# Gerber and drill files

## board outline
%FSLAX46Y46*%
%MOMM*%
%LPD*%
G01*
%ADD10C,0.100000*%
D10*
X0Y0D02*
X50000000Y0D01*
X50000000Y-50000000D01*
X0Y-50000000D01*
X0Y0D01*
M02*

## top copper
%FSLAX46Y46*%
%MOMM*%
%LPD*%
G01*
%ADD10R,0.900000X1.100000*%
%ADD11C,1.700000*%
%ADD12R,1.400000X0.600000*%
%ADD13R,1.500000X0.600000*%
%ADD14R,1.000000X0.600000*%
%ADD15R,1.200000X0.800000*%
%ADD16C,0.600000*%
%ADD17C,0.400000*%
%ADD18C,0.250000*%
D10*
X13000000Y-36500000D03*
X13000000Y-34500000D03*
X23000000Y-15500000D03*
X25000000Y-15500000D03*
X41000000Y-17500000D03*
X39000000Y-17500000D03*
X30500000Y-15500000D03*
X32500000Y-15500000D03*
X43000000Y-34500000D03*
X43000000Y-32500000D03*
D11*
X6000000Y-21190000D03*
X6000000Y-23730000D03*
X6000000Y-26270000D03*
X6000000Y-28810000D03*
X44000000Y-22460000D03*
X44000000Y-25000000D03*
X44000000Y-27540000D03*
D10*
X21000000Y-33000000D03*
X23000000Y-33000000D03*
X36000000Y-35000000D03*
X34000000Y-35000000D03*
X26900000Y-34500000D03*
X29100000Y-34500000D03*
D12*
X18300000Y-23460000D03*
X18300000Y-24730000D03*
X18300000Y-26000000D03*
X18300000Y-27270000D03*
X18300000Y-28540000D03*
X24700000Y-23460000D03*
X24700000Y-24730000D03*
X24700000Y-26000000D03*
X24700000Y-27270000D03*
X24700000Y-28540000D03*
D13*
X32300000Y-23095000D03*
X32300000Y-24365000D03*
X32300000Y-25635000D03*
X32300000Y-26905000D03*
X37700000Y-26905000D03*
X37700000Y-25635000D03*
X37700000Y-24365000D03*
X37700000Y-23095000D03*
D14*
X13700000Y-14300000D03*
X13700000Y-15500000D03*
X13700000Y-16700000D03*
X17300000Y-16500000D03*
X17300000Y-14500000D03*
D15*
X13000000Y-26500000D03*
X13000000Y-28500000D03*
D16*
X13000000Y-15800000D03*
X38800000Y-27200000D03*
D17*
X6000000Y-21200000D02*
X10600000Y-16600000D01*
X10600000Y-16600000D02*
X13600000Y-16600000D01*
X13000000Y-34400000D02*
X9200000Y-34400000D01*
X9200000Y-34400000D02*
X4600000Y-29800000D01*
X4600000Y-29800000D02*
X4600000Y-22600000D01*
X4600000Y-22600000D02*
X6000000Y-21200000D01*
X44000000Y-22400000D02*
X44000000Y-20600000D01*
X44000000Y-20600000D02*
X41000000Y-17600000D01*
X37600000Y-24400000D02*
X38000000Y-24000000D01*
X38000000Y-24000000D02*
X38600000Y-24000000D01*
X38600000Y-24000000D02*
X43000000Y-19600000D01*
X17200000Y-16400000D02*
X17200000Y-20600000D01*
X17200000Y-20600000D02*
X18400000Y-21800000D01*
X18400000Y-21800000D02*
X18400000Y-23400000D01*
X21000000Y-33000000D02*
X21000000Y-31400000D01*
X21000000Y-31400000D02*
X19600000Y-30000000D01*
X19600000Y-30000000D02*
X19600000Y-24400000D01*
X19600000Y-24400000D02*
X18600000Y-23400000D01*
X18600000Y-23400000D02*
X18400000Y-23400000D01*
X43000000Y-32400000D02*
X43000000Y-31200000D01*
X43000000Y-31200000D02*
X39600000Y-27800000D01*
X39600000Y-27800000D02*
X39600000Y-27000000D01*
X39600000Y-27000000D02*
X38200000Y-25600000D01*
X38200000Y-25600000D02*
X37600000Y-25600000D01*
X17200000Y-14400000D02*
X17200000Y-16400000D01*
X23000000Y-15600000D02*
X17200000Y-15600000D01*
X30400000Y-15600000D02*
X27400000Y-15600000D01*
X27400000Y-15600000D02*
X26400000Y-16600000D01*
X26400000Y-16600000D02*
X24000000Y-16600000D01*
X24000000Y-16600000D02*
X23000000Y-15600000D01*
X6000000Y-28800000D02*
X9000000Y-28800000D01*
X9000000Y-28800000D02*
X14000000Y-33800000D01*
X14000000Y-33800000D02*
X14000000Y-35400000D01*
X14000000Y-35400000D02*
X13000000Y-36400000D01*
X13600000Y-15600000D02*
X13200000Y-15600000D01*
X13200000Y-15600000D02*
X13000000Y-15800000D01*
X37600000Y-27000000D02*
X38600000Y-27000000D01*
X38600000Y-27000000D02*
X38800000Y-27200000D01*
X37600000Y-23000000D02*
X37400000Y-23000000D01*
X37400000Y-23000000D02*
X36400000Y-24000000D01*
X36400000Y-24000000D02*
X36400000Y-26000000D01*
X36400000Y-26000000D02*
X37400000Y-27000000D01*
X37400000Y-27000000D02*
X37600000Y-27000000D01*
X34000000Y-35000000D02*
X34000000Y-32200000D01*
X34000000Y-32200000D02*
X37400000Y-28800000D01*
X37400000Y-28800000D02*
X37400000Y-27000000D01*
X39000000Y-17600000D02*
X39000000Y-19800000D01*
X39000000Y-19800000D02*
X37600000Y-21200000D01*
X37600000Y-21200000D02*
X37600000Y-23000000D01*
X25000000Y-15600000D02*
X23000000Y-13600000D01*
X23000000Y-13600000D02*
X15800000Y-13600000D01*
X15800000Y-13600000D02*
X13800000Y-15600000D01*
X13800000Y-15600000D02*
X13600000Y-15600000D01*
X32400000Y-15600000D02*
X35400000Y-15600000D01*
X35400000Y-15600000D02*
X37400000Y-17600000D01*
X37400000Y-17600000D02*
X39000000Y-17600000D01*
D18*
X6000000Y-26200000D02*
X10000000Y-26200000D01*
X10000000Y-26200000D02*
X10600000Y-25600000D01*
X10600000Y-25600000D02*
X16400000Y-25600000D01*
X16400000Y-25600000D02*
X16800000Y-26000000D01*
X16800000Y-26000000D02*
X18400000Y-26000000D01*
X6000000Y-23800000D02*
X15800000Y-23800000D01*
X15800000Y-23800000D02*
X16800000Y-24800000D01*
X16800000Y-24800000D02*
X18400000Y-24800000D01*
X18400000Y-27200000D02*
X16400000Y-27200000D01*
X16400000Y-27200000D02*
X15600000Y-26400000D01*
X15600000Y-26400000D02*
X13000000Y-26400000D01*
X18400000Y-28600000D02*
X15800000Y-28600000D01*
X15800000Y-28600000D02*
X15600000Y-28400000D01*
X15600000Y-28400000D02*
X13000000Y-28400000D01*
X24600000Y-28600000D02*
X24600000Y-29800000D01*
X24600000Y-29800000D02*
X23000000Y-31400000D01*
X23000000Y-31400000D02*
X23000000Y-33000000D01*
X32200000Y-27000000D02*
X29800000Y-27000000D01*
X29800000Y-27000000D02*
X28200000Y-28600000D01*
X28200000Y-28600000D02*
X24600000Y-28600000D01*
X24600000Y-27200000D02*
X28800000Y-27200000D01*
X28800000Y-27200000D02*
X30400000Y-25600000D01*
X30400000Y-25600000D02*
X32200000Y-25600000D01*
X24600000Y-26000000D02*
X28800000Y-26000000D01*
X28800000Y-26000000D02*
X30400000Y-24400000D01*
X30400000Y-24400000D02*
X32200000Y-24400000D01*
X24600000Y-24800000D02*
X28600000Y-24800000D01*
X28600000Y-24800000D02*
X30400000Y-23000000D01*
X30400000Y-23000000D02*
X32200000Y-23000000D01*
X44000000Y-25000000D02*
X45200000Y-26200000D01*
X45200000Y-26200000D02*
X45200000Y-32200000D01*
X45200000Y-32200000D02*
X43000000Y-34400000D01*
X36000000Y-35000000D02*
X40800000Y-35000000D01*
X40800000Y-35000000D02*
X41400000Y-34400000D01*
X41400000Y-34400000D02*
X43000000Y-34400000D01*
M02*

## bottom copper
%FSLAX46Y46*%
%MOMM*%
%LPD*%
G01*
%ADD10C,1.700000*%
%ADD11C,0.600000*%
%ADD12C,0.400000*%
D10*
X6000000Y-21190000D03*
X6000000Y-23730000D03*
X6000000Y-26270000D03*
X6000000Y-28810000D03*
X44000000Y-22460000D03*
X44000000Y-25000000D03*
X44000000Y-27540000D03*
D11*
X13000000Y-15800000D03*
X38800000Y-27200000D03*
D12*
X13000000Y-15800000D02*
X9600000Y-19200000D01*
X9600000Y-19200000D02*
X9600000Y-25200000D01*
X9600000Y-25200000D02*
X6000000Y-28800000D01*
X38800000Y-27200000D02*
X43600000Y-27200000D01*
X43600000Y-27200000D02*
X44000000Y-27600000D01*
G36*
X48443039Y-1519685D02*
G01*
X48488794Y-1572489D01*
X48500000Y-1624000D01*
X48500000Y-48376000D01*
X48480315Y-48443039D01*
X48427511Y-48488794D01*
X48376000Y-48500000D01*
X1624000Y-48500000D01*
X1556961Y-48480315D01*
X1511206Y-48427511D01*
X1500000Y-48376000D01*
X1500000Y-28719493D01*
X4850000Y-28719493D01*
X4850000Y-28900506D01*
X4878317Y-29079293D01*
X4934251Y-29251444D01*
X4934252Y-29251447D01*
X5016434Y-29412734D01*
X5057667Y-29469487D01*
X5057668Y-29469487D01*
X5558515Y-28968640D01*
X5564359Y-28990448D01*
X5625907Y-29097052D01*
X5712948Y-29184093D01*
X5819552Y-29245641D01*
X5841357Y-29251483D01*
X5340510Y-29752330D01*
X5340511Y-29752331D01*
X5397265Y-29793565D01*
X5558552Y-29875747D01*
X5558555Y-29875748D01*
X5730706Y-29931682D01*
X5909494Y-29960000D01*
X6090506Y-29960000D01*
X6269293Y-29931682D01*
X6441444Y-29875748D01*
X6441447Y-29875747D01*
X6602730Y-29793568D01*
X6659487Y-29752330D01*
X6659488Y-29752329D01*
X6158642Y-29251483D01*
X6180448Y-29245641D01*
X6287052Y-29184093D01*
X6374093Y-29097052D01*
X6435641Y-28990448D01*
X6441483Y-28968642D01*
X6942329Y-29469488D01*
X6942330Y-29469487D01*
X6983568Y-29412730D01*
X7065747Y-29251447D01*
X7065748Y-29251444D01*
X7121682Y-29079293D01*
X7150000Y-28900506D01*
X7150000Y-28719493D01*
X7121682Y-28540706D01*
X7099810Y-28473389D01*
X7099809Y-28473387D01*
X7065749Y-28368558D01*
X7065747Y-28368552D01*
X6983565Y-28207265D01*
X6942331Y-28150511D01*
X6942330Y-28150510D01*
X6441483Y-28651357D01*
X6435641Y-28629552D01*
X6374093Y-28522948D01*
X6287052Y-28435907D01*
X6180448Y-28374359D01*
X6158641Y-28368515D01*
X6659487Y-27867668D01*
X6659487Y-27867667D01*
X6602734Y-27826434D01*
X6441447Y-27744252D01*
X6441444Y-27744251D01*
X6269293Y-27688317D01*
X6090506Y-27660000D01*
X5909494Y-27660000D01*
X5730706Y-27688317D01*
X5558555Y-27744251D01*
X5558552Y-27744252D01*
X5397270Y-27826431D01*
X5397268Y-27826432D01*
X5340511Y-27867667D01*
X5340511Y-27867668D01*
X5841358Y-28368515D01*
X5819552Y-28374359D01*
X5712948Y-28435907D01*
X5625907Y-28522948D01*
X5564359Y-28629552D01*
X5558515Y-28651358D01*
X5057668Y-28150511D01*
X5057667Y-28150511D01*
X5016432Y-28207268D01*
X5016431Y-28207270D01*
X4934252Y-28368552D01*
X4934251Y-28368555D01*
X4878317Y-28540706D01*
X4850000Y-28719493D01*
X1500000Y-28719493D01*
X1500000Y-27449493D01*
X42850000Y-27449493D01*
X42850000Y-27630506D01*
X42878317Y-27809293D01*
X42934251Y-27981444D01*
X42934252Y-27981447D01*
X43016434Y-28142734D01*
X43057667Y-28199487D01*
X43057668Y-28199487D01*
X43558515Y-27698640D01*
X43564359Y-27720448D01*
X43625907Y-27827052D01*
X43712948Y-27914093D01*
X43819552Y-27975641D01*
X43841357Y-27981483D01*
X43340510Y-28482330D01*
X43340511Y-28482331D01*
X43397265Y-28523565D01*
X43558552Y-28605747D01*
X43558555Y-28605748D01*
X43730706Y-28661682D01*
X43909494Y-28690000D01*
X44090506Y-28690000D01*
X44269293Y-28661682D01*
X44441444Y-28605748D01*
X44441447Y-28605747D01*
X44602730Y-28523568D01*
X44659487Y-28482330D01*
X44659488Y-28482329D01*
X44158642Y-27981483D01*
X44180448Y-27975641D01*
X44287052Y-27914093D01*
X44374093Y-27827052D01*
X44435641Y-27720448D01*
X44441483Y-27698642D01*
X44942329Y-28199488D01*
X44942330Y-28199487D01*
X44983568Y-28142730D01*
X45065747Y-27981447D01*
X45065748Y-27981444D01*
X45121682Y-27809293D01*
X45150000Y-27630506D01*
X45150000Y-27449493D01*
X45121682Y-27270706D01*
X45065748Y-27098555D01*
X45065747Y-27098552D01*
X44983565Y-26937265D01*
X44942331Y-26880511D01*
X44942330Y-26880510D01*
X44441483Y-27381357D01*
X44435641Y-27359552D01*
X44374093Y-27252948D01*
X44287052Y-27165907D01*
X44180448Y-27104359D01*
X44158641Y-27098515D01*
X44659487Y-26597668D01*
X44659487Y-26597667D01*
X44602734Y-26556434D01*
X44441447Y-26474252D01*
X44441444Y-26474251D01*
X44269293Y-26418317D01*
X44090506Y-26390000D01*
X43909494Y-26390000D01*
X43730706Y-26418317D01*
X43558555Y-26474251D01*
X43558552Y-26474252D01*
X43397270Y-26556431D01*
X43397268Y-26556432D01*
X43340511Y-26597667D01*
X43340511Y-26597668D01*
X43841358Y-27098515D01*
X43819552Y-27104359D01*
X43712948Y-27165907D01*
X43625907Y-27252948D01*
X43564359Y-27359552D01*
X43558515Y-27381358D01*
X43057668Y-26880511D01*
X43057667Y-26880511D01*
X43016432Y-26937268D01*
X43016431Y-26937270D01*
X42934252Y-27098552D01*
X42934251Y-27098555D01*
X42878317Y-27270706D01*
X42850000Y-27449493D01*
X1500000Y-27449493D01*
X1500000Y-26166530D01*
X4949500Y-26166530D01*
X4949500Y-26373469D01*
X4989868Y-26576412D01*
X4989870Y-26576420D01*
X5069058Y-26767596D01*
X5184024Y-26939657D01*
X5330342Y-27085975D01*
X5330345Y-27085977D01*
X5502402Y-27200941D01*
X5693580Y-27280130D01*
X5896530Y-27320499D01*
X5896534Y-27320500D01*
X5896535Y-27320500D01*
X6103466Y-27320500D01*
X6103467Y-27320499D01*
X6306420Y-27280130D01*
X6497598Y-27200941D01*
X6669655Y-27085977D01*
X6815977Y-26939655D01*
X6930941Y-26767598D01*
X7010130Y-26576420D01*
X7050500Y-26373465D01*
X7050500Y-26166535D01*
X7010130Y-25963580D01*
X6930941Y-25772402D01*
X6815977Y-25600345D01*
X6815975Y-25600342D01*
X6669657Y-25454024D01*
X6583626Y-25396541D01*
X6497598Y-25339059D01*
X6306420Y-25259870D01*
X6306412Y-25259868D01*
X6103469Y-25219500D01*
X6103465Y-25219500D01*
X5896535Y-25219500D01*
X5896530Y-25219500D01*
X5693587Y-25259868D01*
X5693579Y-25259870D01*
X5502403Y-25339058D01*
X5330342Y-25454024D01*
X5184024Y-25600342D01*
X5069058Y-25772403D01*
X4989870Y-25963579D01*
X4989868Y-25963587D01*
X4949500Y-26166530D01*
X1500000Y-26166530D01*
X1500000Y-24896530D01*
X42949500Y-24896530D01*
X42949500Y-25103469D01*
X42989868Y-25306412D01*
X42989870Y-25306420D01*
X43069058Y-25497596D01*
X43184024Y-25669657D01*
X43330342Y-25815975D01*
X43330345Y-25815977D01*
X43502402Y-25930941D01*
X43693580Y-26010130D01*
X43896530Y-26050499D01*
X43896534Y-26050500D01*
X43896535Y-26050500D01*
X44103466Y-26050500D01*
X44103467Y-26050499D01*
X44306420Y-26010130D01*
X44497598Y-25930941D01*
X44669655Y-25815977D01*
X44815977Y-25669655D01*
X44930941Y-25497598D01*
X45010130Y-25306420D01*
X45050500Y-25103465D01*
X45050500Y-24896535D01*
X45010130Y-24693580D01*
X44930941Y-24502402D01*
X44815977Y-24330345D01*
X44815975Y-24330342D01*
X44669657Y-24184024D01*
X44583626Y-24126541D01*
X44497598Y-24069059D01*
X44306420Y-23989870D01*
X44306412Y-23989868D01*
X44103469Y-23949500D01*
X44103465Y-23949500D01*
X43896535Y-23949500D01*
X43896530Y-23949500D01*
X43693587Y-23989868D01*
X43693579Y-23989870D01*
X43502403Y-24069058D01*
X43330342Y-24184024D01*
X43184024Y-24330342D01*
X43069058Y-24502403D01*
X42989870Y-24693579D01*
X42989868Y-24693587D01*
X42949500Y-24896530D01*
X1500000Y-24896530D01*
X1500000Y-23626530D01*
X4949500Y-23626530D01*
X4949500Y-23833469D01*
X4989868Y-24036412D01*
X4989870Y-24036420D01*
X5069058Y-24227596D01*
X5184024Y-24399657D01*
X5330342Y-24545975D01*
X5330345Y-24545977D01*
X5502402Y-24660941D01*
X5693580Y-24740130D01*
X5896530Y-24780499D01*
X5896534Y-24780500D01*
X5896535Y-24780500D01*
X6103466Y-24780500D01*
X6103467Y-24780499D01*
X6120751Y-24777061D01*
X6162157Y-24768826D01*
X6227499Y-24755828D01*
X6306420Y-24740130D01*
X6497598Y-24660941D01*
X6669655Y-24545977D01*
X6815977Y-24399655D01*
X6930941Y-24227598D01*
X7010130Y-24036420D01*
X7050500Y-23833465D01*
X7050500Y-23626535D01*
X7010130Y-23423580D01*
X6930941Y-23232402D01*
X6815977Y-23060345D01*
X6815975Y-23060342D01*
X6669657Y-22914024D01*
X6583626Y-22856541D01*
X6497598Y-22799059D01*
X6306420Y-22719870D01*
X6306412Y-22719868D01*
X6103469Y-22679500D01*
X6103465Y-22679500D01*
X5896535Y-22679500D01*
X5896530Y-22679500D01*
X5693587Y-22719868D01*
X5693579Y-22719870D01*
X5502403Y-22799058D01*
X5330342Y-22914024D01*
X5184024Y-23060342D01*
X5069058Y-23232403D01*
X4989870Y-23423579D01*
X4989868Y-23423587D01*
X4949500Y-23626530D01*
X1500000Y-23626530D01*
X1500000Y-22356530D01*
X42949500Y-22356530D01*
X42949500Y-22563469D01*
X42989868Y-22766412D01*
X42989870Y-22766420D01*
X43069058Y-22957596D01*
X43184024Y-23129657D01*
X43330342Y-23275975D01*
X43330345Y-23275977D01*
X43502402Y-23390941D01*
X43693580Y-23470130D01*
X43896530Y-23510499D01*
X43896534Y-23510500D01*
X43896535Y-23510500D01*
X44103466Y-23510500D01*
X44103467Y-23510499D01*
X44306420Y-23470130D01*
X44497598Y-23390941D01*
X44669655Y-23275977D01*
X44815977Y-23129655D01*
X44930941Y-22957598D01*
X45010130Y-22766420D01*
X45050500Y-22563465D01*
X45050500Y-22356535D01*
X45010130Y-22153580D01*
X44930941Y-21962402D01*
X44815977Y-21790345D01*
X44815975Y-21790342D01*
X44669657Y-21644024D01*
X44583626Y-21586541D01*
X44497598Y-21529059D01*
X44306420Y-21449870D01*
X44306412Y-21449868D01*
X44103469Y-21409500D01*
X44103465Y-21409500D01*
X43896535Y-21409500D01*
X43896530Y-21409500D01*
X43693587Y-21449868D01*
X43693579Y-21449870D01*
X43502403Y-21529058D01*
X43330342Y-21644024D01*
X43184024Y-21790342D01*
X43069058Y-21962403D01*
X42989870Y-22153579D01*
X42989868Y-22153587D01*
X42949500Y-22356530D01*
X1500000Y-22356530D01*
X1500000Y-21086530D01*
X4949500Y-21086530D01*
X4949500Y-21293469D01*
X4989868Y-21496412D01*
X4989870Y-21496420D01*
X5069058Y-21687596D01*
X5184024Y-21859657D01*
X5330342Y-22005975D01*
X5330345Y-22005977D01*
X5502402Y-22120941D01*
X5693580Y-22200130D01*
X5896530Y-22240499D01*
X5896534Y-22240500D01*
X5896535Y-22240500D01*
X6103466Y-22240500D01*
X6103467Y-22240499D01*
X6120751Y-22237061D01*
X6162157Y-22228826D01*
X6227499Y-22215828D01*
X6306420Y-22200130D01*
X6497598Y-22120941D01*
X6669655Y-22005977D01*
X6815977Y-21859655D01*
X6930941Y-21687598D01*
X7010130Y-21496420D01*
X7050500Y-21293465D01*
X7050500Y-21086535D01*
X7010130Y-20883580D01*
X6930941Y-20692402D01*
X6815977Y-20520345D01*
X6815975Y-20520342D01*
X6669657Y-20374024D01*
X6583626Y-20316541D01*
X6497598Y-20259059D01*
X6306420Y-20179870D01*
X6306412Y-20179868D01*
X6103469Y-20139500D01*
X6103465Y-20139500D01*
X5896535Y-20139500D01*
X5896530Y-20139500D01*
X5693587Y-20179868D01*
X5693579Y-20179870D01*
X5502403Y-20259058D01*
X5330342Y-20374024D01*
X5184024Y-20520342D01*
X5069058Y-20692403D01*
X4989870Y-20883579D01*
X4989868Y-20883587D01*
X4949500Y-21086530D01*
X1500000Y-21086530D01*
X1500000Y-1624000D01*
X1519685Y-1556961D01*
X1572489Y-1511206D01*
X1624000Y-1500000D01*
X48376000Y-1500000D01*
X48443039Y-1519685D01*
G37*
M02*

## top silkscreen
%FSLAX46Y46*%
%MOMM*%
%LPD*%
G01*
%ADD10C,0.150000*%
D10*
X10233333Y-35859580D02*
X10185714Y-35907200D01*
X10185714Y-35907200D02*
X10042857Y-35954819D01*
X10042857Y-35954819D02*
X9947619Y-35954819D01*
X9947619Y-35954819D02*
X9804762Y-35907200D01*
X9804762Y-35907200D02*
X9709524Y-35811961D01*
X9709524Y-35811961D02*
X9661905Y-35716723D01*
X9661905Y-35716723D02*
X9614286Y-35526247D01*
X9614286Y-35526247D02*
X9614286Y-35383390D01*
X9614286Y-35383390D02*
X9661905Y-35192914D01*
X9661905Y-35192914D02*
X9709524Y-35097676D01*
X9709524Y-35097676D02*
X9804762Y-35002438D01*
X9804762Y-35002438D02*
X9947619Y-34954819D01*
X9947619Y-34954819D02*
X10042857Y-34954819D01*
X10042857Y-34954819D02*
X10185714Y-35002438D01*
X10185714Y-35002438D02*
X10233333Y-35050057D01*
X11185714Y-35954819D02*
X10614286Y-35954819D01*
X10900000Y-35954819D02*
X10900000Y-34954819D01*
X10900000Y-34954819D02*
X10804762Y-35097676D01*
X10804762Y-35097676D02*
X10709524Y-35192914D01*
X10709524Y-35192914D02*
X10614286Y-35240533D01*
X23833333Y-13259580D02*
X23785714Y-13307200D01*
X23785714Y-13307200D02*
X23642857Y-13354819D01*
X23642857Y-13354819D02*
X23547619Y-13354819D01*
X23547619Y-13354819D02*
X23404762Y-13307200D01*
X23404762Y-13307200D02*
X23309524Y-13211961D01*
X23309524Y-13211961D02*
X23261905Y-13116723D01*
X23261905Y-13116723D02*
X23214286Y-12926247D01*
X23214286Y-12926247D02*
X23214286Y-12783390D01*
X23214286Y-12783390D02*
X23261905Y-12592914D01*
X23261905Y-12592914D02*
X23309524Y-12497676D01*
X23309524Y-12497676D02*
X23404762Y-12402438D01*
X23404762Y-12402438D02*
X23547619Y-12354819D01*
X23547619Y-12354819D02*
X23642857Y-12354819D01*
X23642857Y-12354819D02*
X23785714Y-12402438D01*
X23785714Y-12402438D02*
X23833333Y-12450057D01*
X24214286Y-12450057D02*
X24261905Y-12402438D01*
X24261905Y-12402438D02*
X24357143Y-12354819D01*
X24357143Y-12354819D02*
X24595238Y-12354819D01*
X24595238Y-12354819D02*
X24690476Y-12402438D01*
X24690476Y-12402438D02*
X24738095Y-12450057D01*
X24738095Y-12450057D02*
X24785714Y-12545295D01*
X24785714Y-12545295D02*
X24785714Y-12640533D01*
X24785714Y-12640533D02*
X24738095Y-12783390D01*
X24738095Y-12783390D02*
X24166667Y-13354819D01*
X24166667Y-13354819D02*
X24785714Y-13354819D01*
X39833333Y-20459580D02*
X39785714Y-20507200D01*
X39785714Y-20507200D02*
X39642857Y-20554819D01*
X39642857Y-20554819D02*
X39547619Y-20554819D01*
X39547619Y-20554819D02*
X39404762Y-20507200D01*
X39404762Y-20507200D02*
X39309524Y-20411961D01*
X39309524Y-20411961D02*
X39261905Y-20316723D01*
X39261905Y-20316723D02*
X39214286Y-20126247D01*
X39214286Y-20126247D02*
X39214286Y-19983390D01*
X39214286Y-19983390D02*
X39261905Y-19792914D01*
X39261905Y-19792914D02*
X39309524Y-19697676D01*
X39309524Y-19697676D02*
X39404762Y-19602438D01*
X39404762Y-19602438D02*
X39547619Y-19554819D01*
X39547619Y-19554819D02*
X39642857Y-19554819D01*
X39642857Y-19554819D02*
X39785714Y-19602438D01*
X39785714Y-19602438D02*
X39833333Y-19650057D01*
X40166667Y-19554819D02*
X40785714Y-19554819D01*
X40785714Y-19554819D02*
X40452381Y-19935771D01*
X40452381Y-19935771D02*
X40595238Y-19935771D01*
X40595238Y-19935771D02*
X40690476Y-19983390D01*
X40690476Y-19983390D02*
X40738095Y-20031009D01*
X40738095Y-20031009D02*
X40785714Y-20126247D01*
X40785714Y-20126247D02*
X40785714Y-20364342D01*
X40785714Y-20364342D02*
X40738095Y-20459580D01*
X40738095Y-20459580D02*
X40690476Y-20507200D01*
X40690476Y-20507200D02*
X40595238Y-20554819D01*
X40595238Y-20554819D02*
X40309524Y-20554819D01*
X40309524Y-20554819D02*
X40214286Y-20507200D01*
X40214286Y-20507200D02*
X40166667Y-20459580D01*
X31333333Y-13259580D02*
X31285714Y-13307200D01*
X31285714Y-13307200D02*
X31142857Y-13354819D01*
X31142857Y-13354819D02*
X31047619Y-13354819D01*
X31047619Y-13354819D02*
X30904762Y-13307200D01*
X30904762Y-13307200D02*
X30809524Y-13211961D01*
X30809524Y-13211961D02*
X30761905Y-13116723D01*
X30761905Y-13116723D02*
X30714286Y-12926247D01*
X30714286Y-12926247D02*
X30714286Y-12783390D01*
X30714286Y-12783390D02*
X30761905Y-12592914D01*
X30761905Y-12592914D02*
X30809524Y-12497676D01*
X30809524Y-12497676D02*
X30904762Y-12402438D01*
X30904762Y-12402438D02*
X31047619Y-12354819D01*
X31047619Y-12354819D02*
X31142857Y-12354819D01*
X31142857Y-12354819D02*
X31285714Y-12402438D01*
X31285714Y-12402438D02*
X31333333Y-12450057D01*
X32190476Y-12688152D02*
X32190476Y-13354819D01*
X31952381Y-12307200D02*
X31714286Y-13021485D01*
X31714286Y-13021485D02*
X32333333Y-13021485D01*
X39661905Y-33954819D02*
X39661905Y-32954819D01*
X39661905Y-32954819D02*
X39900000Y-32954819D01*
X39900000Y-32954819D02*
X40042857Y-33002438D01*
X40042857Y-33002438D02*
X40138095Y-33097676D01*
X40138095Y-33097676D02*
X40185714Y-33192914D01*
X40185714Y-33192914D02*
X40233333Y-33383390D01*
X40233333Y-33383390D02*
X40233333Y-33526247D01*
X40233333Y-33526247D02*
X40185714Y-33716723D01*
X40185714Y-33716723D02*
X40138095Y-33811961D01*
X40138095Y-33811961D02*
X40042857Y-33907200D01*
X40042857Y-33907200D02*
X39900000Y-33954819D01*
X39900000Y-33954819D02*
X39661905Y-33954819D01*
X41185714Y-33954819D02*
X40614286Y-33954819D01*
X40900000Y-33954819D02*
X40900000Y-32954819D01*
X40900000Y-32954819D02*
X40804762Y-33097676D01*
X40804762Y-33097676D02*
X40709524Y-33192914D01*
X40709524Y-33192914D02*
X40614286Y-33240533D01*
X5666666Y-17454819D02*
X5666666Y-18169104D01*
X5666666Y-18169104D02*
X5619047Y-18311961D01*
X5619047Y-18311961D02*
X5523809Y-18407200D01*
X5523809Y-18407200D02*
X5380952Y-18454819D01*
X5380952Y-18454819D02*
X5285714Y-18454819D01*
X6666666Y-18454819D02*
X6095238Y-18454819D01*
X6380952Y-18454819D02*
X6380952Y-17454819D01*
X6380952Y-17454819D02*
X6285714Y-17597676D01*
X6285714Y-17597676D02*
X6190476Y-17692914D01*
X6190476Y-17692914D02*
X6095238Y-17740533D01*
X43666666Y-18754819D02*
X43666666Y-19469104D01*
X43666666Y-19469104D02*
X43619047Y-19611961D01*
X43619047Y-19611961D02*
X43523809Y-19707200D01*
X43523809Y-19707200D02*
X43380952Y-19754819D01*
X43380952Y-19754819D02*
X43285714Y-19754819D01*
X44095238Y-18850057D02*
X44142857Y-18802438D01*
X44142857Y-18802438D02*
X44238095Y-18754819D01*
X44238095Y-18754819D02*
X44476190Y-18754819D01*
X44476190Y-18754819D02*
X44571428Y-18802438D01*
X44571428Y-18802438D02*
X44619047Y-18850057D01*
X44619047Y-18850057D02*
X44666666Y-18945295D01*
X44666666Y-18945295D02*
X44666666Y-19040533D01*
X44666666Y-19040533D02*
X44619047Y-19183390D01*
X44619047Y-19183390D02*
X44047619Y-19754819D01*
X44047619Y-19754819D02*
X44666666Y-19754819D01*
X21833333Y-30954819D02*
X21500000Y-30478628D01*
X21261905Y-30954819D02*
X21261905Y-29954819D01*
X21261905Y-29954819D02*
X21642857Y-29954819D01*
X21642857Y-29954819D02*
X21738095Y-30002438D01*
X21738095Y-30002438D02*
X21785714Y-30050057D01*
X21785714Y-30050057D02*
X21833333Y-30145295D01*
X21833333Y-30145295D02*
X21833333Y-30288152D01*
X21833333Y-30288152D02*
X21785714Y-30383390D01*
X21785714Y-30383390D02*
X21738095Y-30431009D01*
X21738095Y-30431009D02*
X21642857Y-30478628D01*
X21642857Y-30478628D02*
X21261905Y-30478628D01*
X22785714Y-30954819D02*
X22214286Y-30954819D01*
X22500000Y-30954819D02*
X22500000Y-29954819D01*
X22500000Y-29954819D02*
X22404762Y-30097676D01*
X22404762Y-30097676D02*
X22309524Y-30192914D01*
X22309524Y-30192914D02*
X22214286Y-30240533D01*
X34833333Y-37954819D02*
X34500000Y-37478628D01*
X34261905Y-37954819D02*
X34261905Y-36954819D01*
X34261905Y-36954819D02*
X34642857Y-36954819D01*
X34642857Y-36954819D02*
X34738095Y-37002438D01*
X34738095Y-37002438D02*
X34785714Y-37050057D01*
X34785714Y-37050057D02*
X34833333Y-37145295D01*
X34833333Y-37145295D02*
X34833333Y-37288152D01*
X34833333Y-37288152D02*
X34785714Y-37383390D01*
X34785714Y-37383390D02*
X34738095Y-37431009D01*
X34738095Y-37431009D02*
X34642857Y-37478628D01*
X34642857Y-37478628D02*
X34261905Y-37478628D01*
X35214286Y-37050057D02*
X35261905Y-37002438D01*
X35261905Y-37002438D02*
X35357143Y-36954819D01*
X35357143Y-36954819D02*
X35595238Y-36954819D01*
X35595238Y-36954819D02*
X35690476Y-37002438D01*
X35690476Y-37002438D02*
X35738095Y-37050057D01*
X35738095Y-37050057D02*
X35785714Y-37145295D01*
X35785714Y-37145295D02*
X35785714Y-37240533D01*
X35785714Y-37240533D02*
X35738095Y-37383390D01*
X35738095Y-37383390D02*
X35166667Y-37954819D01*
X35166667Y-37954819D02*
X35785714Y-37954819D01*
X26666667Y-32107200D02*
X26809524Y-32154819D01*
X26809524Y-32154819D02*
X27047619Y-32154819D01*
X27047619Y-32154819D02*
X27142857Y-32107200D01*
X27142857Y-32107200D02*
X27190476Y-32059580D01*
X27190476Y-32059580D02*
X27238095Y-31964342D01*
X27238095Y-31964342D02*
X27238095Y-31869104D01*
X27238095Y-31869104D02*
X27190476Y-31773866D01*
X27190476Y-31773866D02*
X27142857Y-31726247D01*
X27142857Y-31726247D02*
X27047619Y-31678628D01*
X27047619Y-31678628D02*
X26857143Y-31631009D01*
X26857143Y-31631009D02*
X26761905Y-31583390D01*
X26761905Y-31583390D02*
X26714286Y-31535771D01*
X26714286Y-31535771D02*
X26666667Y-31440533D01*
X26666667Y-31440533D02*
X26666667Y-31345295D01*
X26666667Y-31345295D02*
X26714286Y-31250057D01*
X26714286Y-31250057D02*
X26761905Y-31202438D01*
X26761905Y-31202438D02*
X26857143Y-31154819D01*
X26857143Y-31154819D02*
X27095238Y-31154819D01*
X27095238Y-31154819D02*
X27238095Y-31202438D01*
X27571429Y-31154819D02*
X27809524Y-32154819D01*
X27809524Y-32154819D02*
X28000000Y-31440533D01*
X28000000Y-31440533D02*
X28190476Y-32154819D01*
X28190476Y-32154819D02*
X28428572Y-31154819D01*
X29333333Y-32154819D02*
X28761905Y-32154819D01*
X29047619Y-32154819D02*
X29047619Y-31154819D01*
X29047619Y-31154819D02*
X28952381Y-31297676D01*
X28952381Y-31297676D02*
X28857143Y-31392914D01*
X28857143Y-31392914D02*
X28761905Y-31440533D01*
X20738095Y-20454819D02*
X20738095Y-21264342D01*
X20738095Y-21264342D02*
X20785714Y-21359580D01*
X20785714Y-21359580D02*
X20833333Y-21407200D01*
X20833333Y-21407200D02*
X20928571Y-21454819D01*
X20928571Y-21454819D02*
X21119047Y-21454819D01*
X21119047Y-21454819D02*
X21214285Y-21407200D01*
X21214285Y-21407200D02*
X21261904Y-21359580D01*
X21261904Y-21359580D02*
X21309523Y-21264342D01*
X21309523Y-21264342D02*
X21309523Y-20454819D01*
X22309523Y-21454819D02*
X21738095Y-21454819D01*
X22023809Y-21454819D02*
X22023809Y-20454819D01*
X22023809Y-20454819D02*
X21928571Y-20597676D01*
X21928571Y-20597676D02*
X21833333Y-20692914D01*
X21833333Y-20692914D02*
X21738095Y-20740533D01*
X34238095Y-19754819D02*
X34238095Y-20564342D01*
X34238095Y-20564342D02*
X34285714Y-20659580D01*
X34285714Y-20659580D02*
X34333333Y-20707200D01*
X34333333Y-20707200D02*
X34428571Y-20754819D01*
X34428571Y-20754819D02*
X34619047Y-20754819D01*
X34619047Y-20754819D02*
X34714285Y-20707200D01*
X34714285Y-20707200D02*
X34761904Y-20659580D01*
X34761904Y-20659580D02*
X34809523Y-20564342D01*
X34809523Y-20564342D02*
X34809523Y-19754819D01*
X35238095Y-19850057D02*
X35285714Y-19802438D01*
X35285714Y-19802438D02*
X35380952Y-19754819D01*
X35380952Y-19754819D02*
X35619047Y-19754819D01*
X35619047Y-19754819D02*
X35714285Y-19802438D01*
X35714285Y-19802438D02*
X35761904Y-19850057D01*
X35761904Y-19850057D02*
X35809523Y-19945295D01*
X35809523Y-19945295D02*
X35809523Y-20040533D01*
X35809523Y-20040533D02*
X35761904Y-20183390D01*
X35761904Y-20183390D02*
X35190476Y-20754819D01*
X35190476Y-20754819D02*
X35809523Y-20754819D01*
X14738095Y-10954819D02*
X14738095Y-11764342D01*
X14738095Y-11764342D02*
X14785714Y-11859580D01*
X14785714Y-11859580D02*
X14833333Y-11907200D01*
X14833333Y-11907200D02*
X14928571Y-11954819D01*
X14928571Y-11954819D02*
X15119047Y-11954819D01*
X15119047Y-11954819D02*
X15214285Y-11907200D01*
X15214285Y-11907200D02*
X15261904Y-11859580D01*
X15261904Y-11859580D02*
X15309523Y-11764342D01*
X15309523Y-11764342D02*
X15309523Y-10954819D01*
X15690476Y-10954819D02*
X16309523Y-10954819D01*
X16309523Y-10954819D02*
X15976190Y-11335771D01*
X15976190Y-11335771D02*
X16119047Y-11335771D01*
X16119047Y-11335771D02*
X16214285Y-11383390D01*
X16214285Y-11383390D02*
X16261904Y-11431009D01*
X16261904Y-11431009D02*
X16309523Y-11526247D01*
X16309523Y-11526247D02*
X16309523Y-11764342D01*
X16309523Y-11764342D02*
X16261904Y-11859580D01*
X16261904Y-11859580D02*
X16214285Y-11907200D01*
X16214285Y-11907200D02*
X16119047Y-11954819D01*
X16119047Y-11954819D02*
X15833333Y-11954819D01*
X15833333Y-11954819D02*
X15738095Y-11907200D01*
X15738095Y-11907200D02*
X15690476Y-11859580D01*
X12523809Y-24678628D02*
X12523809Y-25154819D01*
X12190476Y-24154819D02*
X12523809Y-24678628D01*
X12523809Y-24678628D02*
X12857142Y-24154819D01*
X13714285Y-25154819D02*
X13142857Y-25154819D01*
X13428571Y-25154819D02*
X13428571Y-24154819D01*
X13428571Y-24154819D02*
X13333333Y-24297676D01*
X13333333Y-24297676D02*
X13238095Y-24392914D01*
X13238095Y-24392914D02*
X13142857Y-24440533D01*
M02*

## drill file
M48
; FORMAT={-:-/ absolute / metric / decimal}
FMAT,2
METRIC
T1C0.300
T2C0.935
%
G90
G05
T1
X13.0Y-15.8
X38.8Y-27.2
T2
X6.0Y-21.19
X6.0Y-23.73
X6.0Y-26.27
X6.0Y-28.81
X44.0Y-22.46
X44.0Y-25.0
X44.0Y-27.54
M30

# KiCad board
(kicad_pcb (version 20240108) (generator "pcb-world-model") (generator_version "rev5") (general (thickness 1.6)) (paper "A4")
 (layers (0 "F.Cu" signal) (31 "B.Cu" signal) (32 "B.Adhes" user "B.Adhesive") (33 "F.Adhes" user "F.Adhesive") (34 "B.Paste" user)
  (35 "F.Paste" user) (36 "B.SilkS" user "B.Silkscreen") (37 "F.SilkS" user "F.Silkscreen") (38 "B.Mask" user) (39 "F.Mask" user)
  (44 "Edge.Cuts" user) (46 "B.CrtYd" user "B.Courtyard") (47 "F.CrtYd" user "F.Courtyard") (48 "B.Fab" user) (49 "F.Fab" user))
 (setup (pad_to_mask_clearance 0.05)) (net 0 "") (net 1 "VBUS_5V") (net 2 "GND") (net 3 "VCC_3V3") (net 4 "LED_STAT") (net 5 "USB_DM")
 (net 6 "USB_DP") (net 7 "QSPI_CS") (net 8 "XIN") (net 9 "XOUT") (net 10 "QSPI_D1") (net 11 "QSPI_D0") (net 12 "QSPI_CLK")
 (gr_rect (start 0.0 0.0) (end 50.0000 50.0000) (stroke (width 0.1) (type default)) (fill none) (layer "Edge.Cuts"))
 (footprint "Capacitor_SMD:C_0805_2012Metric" (layer "F.Cu") (at 13.0000 35.5000 90)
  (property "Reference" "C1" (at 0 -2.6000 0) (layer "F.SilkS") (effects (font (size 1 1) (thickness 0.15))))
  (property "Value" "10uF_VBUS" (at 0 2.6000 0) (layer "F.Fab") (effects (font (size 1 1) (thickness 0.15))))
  (pad "1" smd rect (at -1.0000 0.0000) (size 0.9000 1.1000) (layers "F.Cu" "F.Paste" "F.Mask") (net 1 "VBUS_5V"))
  (pad "2" smd rect (at 1.0000 0.0000) (size 0.9000 1.1000) (layers "F.Cu" "F.Paste" "F.Mask") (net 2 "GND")))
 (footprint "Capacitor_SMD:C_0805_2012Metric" (layer "F.Cu") (at 24.0000 15.5000 0)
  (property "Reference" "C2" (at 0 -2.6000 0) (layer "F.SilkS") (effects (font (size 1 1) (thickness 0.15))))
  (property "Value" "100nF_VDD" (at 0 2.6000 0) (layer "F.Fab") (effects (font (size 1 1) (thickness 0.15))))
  (pad "1" smd rect (at -1.0000 0.0000) (size 0.9000 1.1000) (layers "F.Cu" "F.Paste" "F.Mask") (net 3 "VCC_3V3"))
  (pad "2" smd rect (at 1.0000 0.0000) (size 0.9000 1.1000) (layers "F.Cu" "F.Paste" "F.Mask") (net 2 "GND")))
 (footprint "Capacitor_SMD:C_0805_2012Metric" (layer "F.Cu") (at 40.0000 17.5000 180)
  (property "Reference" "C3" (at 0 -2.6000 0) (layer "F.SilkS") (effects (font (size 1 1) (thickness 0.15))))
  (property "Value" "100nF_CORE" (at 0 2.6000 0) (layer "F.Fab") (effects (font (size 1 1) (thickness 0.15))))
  (pad "1" smd rect (at -1.0000 0.0000) (size 0.9000 1.1000) (layers "F.Cu" "F.Paste" "F.Mask") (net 3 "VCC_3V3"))
  (pad "2" smd rect (at 1.0000 0.0000) (size 0.9000 1.1000) (layers "F.Cu" "F.Paste" "F.Mask") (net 2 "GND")))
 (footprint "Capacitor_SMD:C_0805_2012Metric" (layer "F.Cu") (at 31.5000 15.5000 0)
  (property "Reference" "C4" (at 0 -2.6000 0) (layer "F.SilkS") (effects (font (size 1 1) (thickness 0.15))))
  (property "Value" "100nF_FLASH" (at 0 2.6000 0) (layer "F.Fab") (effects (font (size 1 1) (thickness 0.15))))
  (pad "1" smd rect (at -1.0000 0.0000) (size 0.9000 1.1000) (layers "F.Cu" "F.Paste" "F.Mask") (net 3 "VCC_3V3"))
  (pad "2" smd rect (at 1.0000 0.0000) (size 0.9000 1.1000) (layers "F.Cu" "F.Paste" "F.Mask") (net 2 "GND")))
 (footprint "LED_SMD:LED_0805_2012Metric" (layer "F.Cu") (at 43.0000 33.5000 90)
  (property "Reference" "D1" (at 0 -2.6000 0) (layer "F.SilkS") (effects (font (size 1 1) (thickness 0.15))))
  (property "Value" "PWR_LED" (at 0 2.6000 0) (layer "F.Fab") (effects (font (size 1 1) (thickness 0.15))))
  (pad "1" smd rect (at -1.0000 0.0000) (size 0.9000 1.1000) (layers "F.Cu" "F.Paste" "F.Mask") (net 3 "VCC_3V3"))
  (pad "2" smd rect (at 1.0000 0.0000) (size 0.9000 1.1000) (layers "F.Cu" "F.Paste" "F.Mask") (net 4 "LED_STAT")))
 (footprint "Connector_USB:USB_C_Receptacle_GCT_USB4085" (layer "F.Cu") (at 6.0000 25.0000 0) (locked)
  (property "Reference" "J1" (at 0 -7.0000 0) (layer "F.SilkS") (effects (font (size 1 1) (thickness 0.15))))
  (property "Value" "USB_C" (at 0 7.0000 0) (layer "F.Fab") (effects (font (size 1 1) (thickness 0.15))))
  (pad "1" thru_hole circle (at 0.0000 -3.8100) (size 1.7000 1.7000) (drill 0.9350) (layers "*.Cu" "*.Mask") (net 1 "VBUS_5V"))
  (pad "2" thru_hole circle (at 0.0000 -1.2700) (size 1.7000 1.7000) (drill 0.9350) (layers "*.Cu" "*.Mask") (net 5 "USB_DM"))
  (pad "3" thru_hole circle (at 0.0000 1.2700) (size 1.7000 1.7000) (drill 0.9350) (layers "*.Cu" "*.Mask") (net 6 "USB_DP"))
  (pad "4" thru_hole circle (at 0.0000 3.8100) (size 1.7000 1.7000) (drill 0.9350) (layers "*.Cu" "*.Mask") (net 2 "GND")))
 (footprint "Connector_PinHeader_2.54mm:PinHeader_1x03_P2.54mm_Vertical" (layer "F.Cu") (at 44.0000 25.0000 0) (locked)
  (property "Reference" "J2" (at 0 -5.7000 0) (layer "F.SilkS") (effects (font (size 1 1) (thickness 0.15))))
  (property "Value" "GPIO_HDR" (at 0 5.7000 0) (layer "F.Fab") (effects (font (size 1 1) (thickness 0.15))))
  (pad "1" thru_hole circle (at 0.0000 -2.5400) (size 1.7000 1.7000) (drill 0.9350) (layers "*.Cu" "*.Mask") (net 3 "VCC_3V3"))
  (pad "2" thru_hole circle (at 0.0000 0.0000) (size 1.7000 1.7000) (drill 0.9350) (layers "*.Cu" "*.Mask") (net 4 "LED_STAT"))
  (pad "3" thru_hole circle (at 0.0000 2.5400) (size 1.7000 1.7000) (drill 0.9350) (layers "*.Cu" "*.Mask") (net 2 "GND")))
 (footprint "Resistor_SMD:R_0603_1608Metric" (layer "F.Cu") (at 22.0000 33.0000 0)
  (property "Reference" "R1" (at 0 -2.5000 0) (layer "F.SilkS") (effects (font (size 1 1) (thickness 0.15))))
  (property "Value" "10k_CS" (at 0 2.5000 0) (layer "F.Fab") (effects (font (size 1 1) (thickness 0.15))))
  (pad "1" smd rect (at -1.0000 0.0000) (size 0.9000 1.1000) (layers "F.Cu" "F.Paste" "F.Mask") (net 3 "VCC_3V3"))
  (pad "2" smd rect (at 1.0000 0.0000) (size 0.9000 1.1000) (layers "F.Cu" "F.Paste" "F.Mask") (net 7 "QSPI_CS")))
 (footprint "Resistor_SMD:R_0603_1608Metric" (layer "F.Cu") (at 35.0000 35.0000 180)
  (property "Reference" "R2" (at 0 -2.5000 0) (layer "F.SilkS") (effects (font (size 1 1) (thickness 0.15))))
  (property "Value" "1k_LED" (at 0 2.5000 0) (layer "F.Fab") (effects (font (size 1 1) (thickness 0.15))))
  (pad "1" smd rect (at -1.0000 0.0000) (size 0.9000 1.1000) (layers "F.Cu" "F.Paste" "F.Mask") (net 4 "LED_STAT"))
  (pad "2" smd rect (at 1.0000 0.0000) (size 0.9000 1.1000) (layers "F.Cu" "F.Paste" "F.Mask") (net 2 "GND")))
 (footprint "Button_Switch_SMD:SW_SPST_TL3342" (layer "F.Cu") (at 28.0000 34.5000 0)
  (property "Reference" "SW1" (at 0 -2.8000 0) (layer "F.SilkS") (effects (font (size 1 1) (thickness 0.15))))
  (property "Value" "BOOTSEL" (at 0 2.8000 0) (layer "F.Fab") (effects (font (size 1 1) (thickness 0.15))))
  (pad "1" smd rect (at -1.1000 0.0000) (size 0.9000 1.1000) (layers "F.Cu" "F.Paste" "F.Mask") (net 7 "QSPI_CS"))
  (pad "2" smd rect (at 1.1000 0.0000) (size 0.9000 1.1000) (layers "F.Cu" "F.Paste" "F.Mask") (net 2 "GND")))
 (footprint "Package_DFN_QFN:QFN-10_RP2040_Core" (layer "F.Cu") (at 21.5000 26.0000 0)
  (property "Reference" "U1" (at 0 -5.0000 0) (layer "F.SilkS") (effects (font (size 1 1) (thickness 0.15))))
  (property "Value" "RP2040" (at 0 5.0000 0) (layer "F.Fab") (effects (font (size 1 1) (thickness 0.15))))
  (pad "1" smd rect (at -3.2000 -2.5400) (size 1.4000 0.6000) (layers "F.Cu" "F.Paste" "F.Mask") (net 3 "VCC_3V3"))
  (pad "2" smd rect (at -3.2000 -1.2700) (size 1.4000 0.6000) (layers "F.Cu" "F.Paste" "F.Mask") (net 5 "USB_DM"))
  (pad "3" smd rect (at -3.2000 0.0000) (size 1.4000 0.6000) (layers "F.Cu" "F.Paste" "F.Mask") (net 6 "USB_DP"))
  (pad "4" smd rect (at -3.2000 1.2700) (size 1.4000 0.6000) (layers "F.Cu" "F.Paste" "F.Mask") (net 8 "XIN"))
  (pad "5" smd rect (at -3.2000 2.5400) (size 1.4000 0.6000) (layers "F.Cu" "F.Paste" "F.Mask") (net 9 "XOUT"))
  (pad "6" smd rect (at 3.2000 -2.5400) (size 1.4000 0.6000) (layers "F.Cu" "F.Paste" "F.Mask") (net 4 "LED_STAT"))
  (pad "7" smd rect (at 3.2000 -1.2700) (size 1.4000 0.6000) (layers "F.Cu" "F.Paste" "F.Mask") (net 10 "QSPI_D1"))
  (pad "8" smd rect (at 3.2000 0.0000) (size 1.4000 0.6000) (layers "F.Cu" "F.Paste" "F.Mask") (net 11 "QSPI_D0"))
  (pad "9" smd rect (at 3.2000 1.2700) (size 1.4000 0.6000) (layers "F.Cu" "F.Paste" "F.Mask") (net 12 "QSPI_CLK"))
  (pad "10" smd rect (at 3.2000 2.5400) (size 1.4000 0.6000) (layers "F.Cu" "F.Paste" "F.Mask") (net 7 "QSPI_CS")))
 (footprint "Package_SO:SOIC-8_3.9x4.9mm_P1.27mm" (layer "F.Cu") (at 35.0000 25.0000 0)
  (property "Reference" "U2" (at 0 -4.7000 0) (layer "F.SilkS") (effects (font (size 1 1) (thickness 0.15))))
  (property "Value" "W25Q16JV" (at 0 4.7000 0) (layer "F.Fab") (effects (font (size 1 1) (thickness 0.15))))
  (pad "1" smd rect (at -2.7000 -1.9050) (size 1.5000 0.6000) (layers "F.Cu" "F.Paste" "F.Mask") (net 10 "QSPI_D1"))
  (pad "2" smd rect (at -2.7000 -0.6350) (size 1.5000 0.6000) (layers "F.Cu" "F.Paste" "F.Mask") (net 11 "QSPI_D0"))
  (pad "3" smd rect (at -2.7000 0.6350) (size 1.5000 0.6000) (layers "F.Cu" "F.Paste" "F.Mask") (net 12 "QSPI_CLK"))
  (pad "4" smd rect (at -2.7000 1.9050) (size 1.5000 0.6000) (layers "F.Cu" "F.Paste" "F.Mask") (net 7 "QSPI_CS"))
  (pad "5" smd rect (at 2.7000 1.9050) (size 1.5000 0.6000) (layers "F.Cu" "F.Paste" "F.Mask") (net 2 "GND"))
  (pad "6" smd rect (at 2.7000 0.6350) (size 1.5000 0.6000) (layers "F.Cu" "F.Paste" "F.Mask") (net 3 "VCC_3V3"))
  (pad "7" smd rect (at 2.7000 -0.6350) (size 1.5000 0.6000) (layers "F.Cu" "F.Paste" "F.Mask") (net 3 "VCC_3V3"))
  (pad "8" smd rect (at 2.7000 -1.9050) (size 1.5000 0.6000) (layers "F.Cu" "F.Paste" "F.Mask") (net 2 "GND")))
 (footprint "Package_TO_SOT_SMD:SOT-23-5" (layer "F.Cu") (at 15.5000 15.5000 0)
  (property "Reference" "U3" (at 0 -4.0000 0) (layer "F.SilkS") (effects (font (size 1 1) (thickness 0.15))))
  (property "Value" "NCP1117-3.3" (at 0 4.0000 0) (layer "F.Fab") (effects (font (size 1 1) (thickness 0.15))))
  (pad "1" smd rect (at -1.8000 -1.2000) (size 1.0000 0.6000) (layers "F.Cu" "F.Paste" "F.Mask") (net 1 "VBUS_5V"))
  (pad "2" smd rect (at -1.8000 0.0000) (size 1.0000 0.6000) (layers "F.Cu" "F.Paste" "F.Mask") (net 2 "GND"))
  (pad "3" smd rect (at -1.8000 1.2000) (size 1.0000 0.6000) (layers "F.Cu" "F.Paste" "F.Mask") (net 1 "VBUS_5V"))
  (pad "4" smd rect (at 1.8000 1.0000) (size 1.0000 0.6000) (layers "F.Cu" "F.Paste" "F.Mask") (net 3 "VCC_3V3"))
  (pad "5" smd rect (at 1.8000 -1.0000) (size 1.0000 0.6000) (layers "F.Cu" "F.Paste" "F.Mask") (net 3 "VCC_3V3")))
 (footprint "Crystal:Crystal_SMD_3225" (layer "F.Cu") (at 13.0000 27.5000 0)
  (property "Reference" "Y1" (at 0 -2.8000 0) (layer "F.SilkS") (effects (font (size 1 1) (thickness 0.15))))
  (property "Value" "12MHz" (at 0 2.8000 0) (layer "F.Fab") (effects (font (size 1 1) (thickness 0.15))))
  (pad "1" smd rect (at 0.0000 -1.0000) (size 1.2000 0.8000) (layers "F.Cu" "F.Paste" "F.Mask") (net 8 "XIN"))
  (pad "2" smd rect (at 0.0000 1.0000) (size 1.2000 0.8000) (layers "F.Cu" "F.Paste" "F.Mask") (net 9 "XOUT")))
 (segment (start 6.0000 21.2000) (end 10.6000 16.6000) (width 0.4000) (layer "F.Cu") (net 1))
 (segment (start 10.6000 16.6000) (end 13.6000 16.6000) (width 0.4000) (layer "F.Cu") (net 1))
 (segment (start 13.0000 34.4000) (end 9.2000 34.4000) (width 0.4000) (layer "F.Cu") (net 1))
 (segment (start 9.2000 34.4000) (end 4.6000 29.8000) (width 0.4000) (layer "F.Cu") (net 1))
 (segment (start 4.6000 29.8000) (end 4.6000 22.6000) (width 0.4000) (layer "F.Cu") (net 1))
 (segment (start 4.6000 22.6000) (end 6.0000 21.2000) (width 0.4000) (layer "F.Cu") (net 1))
 (segment (start 44.0000 22.4000) (end 44.0000 20.6000) (width 0.4000) (layer "F.Cu") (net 3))
 (segment (start 44.0000 20.6000) (end 41.0000 17.6000) (width 0.4000) (layer "F.Cu") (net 3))
 (segment (start 37.6000 24.4000) (end 38.0000 24.0000) (width 0.4000) (layer "F.Cu") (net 3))
 (segment (start 38.0000 24.0000) (end 38.6000 24.0000) (width 0.4000) (layer "F.Cu") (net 3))
 (segment (start 38.6000 24.0000) (end 43.0000 19.6000) (width 0.4000) (layer "F.Cu") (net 3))
 (segment (start 17.2000 16.4000) (end 17.2000 20.6000) (width 0.4000) (layer "F.Cu") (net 3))
 (segment (start 17.2000 20.6000) (end 18.4000 21.8000) (width 0.4000) (layer "F.Cu") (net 3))
 (segment (start 18.4000 21.8000) (end 18.4000 23.4000) (width 0.4000) (layer "F.Cu") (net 3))
 (segment (start 21.0000 33.0000) (end 21.0000 31.4000) (width 0.4000) (layer "F.Cu") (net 3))
 (segment (start 21.0000 31.4000) (end 19.6000 30.0000) (width 0.4000) (layer "F.Cu") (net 3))
 (segment (start 19.6000 30.0000) (end 19.6000 24.4000) (width 0.4000) (layer "F.Cu") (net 3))
 (segment (start 19.6000 24.4000) (end 18.6000 23.4000) (width 0.4000) (layer "F.Cu") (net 3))
 (segment (start 18.6000 23.4000) (end 18.4000 23.4000) (width 0.4000) (layer "F.Cu") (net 3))
 (segment (start 43.0000 32.4000) (end 43.0000 31.2000) (width 0.4000) (layer "F.Cu") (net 3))
 (segment (start 43.0000 31.2000) (end 39.6000 27.8000) (width 0.4000) (layer "F.Cu") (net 3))
 (segment (start 39.6000 27.8000) (end 39.6000 27.0000) (width 0.4000) (layer "F.Cu") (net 3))
 (segment (start 39.6000 27.0000) (end 38.2000 25.6000) (width 0.4000) (layer "F.Cu") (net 3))
 (segment (start 38.2000 25.6000) (end 37.6000 25.6000) (width 0.4000) (layer "F.Cu") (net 3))
 (segment (start 17.2000 14.4000) (end 17.2000 16.4000) (width 0.4000) (layer "F.Cu") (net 3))
 (segment (start 23.0000 15.6000) (end 17.2000 15.6000) (width 0.4000) (layer "F.Cu") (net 3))
 (segment (start 30.4000 15.6000) (end 27.4000 15.6000) (width 0.4000) (layer "F.Cu") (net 3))
 (segment (start 27.4000 15.6000) (end 26.4000 16.6000) (width 0.4000) (layer "F.Cu") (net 3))
 (segment (start 26.4000 16.6000) (end 24.0000 16.6000) (width 0.4000) (layer "F.Cu") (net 3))
 (segment (start 24.0000 16.6000) (end 23.0000 15.6000) (width 0.4000) (layer "F.Cu") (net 3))
 (segment (start 6.0000 28.8000) (end 9.0000 28.8000) (width 0.4000) (layer "F.Cu") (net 2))
 (segment (start 9.0000 28.8000) (end 14.0000 33.8000) (width 0.4000) (layer "F.Cu") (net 2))
 (segment (start 14.0000 33.8000) (end 14.0000 35.4000) (width 0.4000) (layer "F.Cu") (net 2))
 (segment (start 14.0000 35.4000) (end 13.0000 36.4000) (width 0.4000) (layer "F.Cu") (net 2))
 (segment (start 13.6000 15.6000) (end 13.2000 15.6000) (width 0.4000) (layer "F.Cu") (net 2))
 (segment (start 13.2000 15.6000) (end 13.0000 15.8000) (width 0.4000) (layer "F.Cu") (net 2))
 (segment (start 13.0000 15.8000) (end 9.6000 19.2000) (width 0.4000) (layer "B.Cu") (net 2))
 (segment (start 9.6000 19.2000) (end 9.6000 25.2000) (width 0.4000) (layer "B.Cu") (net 2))
 (segment (start 9.6000 25.2000) (end 6.0000 28.8000) (width 0.4000) (layer "B.Cu") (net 2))
 (segment (start 37.6000 27.0000) (end 38.6000 27.0000) (width 0.4000) (layer "F.Cu") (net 2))
 (segment (start 38.6000 27.0000) (end 38.8000 27.2000) (width 0.4000) (layer "F.Cu") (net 2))
 (segment (start 38.8000 27.2000) (end 43.6000 27.2000) (width 0.4000) (layer "B.Cu") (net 2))
 (segment (start 43.6000 27.2000) (end 44.0000 27.6000) (width 0.4000) (layer "B.Cu") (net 2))
 (segment (start 37.6000 23.0000) (end 37.4000 23.0000) (width 0.4000) (layer "F.Cu") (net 2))
 (segment (start 37.4000 23.0000) (end 36.4000 24.0000) (width 0.4000) (layer "F.Cu") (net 2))
 (segment (start 36.4000 24.0000) (end 36.4000 26.0000) (width 0.4000) (layer "F.Cu") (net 2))
 (segment (start 36.4000 26.0000) (end 37.4000 27.0000) (width 0.4000) (layer "F.Cu") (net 2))
 (segment (start 37.4000 27.0000) (end 37.6000 27.0000) (width 0.4000) (layer "F.Cu") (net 2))
 (segment (start 34.0000 35.0000) (end 34.0000 32.2000) (width 0.4000) (layer "F.Cu") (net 2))
 (segment (start 34.0000 32.2000) (end 37.4000 28.8000) (width 0.4000) (layer "F.Cu") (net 2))
 (segment (start 37.4000 28.8000) (end 37.4000 27.0000) (width 0.4000) (layer "F.Cu") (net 2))
 (segment (start 39.0000 17.6000) (end 39.0000 19.8000) (width 0.4000) (layer "F.Cu") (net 2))
 (segment (start 39.0000 19.8000) (end 37.6000 21.2000) (width 0.4000) (layer "F.Cu") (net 2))
 (segment (start 37.6000 21.2000) (end 37.6000 23.0000) (width 0.4000) (layer "F.Cu") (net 2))
 (segment (start 25.0000 15.6000) (end 23.0000 13.6000) (width 0.4000) (layer "F.Cu") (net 2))
 (segment (start 23.0000 13.6000) (end 15.8000 13.6000) (width 0.4000) (layer "F.Cu") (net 2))
 (segment (start 15.8000 13.6000) (end 13.8000 15.6000) (width 0.4000) (layer "F.Cu") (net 2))
 (segment (start 13.8000 15.6000) (end 13.6000 15.6000) (width 0.4000) (layer "F.Cu") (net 2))
 (segment (start 32.4000 15.6000) (end 35.4000 15.6000) (width 0.4000) (layer "F.Cu") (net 2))
 (segment (start 35.4000 15.6000) (end 37.4000 17.6000) (width 0.4000) (layer "F.Cu") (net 2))
 (segment (start 37.4000 17.6000) (end 39.0000 17.6000) (width 0.4000) (layer "F.Cu") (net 2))
 (segment (start 6.0000 26.2000) (end 10.0000 26.2000) (width 0.2500) (layer "F.Cu") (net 6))
 (segment (start 10.0000 26.2000) (end 10.6000 25.6000) (width 0.2500) (layer "F.Cu") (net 6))
 (segment (start 10.6000 25.6000) (end 16.4000 25.6000) (width 0.2500) (layer "F.Cu") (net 6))
 (segment (start 16.4000 25.6000) (end 16.8000 26.0000) (width 0.2500) (layer "F.Cu") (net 6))
 (segment (start 16.8000 26.0000) (end 18.4000 26.0000) (width 0.2500) (layer "F.Cu") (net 6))
 (segment (start 6.0000 23.8000) (end 15.8000 23.8000) (width 0.2500) (layer "F.Cu") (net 5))
 (segment (start 15.8000 23.8000) (end 16.8000 24.8000) (width 0.2500) (layer "F.Cu") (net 5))
 (segment (start 16.8000 24.8000) (end 18.4000 24.8000) (width 0.2500) (layer "F.Cu") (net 5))
 (segment (start 18.4000 27.2000) (end 16.4000 27.2000) (width 0.2500) (layer "F.Cu") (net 8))
 (segment (start 16.4000 27.2000) (end 15.6000 26.4000) (width 0.2500) (layer "F.Cu") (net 8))
 (segment (start 15.6000 26.4000) (end 13.0000 26.4000) (width 0.2500) (layer "F.Cu") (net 8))
 (segment (start 18.4000 28.6000) (end 15.8000 28.6000) (width 0.2500) (layer "F.Cu") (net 9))
 (segment (start 15.8000 28.6000) (end 15.6000 28.4000) (width 0.2500) (layer "F.Cu") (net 9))
 (segment (start 15.6000 28.4000) (end 13.0000 28.4000) (width 0.2500) (layer "F.Cu") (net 9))
 (segment (start 24.6000 28.6000) (end 24.6000 29.8000) (width 0.2500) (layer "F.Cu") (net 7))
 (segment (start 24.6000 29.8000) (end 23.0000 31.4000) (width 0.2500) (layer "F.Cu") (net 7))
 (segment (start 23.0000 31.4000) (end 23.0000 33.0000) (width 0.2500) (layer "F.Cu") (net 7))
 (segment (start 32.2000 27.0000) (end 29.8000 27.0000) (width 0.2500) (layer "F.Cu") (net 7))
 (segment (start 29.8000 27.0000) (end 28.2000 28.6000) (width 0.2500) (layer "F.Cu") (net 7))
 (segment (start 28.2000 28.6000) (end 24.6000 28.6000) (width 0.2500) (layer "F.Cu") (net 7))
 (segment (start 24.6000 27.2000) (end 28.8000 27.2000) (width 0.2500) (layer "F.Cu") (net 12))
 (segment (start 28.8000 27.2000) (end 30.4000 25.6000) (width 0.2500) (layer "F.Cu") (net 12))
 (segment (start 30.4000 25.6000) (end 32.2000 25.6000) (width 0.2500) (layer "F.Cu") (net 12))
 (segment (start 24.6000 26.0000) (end 28.8000 26.0000) (width 0.2500) (layer "F.Cu") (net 11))
 (segment (start 28.8000 26.0000) (end 30.4000 24.4000) (width 0.2500) (layer "F.Cu") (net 11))
 (segment (start 30.4000 24.4000) (end 32.2000 24.4000) (width 0.2500) (layer "F.Cu") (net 11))
 (segment (start 24.6000 24.8000) (end 28.6000 24.8000) (width 0.2500) (layer "F.Cu") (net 10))
 (segment (start 28.6000 24.8000) (end 30.4000 23.0000) (width 0.2500) (layer "F.Cu") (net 10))
 (segment (start 30.4000 23.0000) (end 32.2000 23.0000) (width 0.2500) (layer "F.Cu") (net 10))
 (segment (start 44.0000 25.0000) (end 45.2000 26.2000) (width 0.2500) (layer "F.Cu") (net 4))
 (segment (start 45.2000 26.2000) (end 45.2000 32.2000) (width 0.2500) (layer "F.Cu") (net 4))
 (segment (start 45.2000 32.2000) (end 43.0000 34.4000) (width 0.2500) (layer "F.Cu") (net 4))
 (segment (start 36.0000 35.0000) (end 40.8000 35.0000) (width 0.2500) (layer "F.Cu") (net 4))
 (segment (start 40.8000 35.0000) (end 41.4000 34.4000) (width 0.2500) (layer "F.Cu") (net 4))
 (segment (start 41.4000 34.4000) (end 43.0000 34.4000) (width 0.2500) (layer "F.Cu") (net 4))
 (via (at 13.0000 15.8000) (size 0.6000) (drill 0.3000) (layers "F.Cu" "B.Cu") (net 2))
 (via (at 38.8000 27.2000) (size 0.6000) (drill 0.3000) (layers "F.Cu" "B.Cu") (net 2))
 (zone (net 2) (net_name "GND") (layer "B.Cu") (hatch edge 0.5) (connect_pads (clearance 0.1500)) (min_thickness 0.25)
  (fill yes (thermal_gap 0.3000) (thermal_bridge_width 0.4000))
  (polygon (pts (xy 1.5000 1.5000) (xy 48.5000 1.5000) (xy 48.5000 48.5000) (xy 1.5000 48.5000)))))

